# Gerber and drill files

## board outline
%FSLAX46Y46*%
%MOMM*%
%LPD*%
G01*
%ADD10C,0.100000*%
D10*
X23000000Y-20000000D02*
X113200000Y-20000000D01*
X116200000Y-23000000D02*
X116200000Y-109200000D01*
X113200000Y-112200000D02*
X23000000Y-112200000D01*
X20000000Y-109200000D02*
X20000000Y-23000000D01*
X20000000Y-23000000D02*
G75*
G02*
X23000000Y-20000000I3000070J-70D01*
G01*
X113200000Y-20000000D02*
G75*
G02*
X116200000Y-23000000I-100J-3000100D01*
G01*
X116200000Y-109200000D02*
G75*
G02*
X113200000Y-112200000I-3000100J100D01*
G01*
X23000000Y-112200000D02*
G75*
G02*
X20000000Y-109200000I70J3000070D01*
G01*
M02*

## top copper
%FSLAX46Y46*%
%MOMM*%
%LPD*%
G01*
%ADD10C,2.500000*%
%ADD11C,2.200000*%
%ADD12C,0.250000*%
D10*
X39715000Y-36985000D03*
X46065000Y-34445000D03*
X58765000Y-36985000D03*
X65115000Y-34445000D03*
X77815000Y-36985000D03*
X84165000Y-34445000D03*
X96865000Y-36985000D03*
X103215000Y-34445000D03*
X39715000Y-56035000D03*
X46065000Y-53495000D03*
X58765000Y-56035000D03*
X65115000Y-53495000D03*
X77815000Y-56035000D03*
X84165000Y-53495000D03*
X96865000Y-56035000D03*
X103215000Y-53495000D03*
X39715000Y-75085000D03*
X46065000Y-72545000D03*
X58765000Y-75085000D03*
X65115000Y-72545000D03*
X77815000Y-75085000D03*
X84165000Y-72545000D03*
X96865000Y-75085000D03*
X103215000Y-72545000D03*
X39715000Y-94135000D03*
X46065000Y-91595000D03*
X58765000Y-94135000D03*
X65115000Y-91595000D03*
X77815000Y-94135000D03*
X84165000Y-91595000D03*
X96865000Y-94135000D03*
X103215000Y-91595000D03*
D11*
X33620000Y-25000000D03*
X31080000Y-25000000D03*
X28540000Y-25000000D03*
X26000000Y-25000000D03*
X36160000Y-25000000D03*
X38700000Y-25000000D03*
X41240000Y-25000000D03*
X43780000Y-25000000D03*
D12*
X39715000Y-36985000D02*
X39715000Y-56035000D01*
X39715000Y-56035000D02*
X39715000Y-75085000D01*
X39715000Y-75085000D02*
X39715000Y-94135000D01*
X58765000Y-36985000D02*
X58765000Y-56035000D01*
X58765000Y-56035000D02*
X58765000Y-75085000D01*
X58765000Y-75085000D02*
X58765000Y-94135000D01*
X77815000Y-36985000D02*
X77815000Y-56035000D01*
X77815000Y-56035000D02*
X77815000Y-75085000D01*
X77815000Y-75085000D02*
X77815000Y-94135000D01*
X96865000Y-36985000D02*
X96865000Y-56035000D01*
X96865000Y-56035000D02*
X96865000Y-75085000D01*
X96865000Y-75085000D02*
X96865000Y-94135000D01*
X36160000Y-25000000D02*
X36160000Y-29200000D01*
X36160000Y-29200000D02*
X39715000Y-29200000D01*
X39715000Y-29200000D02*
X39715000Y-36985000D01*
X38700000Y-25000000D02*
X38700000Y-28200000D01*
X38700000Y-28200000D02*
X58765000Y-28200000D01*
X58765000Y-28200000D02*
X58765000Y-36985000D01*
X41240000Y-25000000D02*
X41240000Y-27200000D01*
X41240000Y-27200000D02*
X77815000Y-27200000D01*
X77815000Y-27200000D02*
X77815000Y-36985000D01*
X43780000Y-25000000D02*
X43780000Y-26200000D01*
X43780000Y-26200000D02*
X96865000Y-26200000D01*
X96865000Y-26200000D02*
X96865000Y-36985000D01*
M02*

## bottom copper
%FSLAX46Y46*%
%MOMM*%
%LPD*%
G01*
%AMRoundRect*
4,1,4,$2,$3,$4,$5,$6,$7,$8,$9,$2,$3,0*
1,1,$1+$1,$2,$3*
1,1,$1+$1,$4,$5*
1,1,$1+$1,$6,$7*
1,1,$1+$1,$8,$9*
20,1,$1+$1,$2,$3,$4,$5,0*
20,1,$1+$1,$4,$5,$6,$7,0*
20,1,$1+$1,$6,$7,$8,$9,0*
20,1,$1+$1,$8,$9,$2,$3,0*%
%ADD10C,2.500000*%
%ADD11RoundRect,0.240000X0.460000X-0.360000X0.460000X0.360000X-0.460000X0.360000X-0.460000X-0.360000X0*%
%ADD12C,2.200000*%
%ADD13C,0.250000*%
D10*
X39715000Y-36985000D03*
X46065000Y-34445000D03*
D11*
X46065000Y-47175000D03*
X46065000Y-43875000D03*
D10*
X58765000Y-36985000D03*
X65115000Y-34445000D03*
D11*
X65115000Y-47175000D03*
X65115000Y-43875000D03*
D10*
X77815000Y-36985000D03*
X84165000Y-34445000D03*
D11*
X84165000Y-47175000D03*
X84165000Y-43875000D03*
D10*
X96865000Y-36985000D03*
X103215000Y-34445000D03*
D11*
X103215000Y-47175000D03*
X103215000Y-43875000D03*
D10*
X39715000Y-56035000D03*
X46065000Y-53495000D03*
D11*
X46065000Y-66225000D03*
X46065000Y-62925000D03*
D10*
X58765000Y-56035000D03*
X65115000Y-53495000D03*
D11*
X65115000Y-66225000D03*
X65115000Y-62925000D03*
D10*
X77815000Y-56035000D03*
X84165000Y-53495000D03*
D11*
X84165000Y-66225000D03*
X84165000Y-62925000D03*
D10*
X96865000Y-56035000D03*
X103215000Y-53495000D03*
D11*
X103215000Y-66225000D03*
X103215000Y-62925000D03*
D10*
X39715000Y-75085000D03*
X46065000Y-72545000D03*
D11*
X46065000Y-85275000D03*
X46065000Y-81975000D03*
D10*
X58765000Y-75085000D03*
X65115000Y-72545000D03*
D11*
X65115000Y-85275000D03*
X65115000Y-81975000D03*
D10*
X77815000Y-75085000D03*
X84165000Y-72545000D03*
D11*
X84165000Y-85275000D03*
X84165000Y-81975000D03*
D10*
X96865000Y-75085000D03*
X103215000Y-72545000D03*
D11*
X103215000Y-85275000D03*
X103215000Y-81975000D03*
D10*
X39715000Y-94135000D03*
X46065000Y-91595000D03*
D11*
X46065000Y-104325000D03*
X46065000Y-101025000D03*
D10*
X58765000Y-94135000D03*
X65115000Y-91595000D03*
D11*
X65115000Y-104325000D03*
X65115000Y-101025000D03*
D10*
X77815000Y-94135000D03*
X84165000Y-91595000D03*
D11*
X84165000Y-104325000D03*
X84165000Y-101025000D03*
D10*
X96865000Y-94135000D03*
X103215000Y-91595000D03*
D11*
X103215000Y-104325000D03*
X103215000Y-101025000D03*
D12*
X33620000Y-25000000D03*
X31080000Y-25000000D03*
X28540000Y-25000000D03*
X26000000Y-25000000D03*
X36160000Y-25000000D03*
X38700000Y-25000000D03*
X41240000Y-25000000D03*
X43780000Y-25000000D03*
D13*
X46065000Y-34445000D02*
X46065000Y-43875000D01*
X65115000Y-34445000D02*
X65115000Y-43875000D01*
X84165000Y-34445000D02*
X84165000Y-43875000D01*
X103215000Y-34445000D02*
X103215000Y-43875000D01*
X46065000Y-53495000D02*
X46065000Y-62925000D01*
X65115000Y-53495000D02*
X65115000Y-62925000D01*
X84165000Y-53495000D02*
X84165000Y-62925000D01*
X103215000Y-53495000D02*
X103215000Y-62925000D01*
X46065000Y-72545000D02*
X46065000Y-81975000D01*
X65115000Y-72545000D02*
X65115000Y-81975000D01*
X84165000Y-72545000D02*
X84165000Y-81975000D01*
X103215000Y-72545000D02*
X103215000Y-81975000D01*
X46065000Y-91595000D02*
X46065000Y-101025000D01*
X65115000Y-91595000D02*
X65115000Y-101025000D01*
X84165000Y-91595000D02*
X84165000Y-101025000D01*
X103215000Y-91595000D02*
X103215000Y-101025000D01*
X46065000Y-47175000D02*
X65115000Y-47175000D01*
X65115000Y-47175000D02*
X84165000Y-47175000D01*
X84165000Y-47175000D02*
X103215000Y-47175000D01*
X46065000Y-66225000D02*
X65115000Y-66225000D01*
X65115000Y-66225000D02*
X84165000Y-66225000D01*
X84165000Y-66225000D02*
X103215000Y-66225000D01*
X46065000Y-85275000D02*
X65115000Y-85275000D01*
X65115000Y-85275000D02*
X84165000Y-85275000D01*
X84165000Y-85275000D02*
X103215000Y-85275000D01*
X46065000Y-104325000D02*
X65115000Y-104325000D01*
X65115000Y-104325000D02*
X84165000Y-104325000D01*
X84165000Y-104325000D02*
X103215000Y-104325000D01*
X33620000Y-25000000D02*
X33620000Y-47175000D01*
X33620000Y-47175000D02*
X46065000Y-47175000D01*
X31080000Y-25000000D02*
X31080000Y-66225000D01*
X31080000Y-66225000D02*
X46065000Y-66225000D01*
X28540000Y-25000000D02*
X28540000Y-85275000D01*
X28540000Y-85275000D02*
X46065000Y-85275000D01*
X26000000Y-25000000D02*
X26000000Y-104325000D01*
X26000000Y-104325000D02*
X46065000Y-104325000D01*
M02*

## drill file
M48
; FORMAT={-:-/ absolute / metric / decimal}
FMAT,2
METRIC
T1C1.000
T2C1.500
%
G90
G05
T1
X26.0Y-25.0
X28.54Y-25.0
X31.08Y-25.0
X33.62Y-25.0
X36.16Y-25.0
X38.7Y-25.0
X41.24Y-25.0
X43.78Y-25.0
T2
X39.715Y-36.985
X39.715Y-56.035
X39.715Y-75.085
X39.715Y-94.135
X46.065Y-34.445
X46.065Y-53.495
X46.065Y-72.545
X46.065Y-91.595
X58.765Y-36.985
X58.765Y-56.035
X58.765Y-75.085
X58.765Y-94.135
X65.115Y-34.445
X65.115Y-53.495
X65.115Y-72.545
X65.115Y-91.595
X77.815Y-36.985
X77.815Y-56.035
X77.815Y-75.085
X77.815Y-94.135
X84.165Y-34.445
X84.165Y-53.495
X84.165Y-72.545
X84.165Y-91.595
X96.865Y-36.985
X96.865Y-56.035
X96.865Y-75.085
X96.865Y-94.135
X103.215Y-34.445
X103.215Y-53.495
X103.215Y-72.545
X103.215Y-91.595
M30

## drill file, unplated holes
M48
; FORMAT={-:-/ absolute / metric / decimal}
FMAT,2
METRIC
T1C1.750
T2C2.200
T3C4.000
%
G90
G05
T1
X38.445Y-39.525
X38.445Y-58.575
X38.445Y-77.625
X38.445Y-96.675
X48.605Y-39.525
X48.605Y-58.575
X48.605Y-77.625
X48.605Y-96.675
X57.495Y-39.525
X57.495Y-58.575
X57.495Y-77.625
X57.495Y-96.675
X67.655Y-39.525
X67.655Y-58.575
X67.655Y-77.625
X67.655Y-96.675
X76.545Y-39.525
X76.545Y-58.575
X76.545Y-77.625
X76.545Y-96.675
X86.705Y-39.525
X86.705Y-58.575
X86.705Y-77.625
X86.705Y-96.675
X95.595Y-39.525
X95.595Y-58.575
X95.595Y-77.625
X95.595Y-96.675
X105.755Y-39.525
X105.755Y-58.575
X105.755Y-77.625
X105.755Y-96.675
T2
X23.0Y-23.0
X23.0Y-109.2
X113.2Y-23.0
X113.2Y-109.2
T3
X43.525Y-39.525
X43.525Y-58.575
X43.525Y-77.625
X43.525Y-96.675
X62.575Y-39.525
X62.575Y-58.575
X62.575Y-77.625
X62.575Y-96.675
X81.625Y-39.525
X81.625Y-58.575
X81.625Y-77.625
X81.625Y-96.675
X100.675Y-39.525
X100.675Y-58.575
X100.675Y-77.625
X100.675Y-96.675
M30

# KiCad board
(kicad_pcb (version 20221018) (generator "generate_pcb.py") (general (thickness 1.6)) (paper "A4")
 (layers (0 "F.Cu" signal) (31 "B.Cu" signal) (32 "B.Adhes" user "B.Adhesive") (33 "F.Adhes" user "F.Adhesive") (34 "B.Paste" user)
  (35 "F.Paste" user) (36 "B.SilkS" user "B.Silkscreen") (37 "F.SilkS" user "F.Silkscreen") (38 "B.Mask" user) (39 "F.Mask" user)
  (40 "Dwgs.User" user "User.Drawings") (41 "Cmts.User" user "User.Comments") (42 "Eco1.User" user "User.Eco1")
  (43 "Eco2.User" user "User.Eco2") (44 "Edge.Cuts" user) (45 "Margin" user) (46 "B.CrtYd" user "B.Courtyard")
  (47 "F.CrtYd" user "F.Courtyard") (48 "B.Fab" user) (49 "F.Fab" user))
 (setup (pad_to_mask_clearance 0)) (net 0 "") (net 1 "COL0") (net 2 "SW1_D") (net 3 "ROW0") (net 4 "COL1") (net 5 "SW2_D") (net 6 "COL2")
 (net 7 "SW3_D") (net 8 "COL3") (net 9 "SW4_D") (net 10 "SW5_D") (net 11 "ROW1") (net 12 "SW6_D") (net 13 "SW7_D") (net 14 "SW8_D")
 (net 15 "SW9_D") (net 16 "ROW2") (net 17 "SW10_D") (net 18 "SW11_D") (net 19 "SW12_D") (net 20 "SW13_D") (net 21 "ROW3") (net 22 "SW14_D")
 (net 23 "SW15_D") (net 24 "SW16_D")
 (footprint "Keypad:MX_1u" (layer "F.Cu") (at 43.5250 39.5250)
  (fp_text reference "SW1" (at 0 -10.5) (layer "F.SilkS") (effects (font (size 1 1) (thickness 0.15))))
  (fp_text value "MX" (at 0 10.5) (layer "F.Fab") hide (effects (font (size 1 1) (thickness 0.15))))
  (pad "1" thru_hole circle (at -3.81 -2.54) (size 2.5 2.5) (drill 1.5) (layers "*.Cu" "*.Mask") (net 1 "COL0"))
  (pad "2" thru_hole circle (at 2.54 -5.08) (size 2.5 2.5) (drill 1.5) (layers "*.Cu" "*.Mask") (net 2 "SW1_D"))
  (pad "" np_thru_hole circle (at 0 0) (size 4 4) (drill 4) (layers "*.Cu" "*.Mask"))
  (pad "" np_thru_hole circle (at -5.08 0) (size 1.75 1.75) (drill 1.75) (layers "*.Cu" "*.Mask"))
  (pad "" np_thru_hole circle (at 5.08 0) (size 1.75 1.75) (drill 1.75) (layers "*.Cu" "*.Mask")))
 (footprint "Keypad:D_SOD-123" (layer "B.Cu") (at 46.0650 45.5250 90)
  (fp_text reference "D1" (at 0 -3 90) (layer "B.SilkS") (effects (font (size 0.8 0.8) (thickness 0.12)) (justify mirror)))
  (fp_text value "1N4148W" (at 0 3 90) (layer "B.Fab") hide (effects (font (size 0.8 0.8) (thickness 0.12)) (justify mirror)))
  (pad "1" smd roundrect (at -1.65 0 90) (size 1.2 1.4) (layers "B.Cu" "B.Paste" "B.Mask") (roundrect_rratio 0.2) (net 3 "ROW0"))
  (pad "2" smd roundrect (at 1.65 0 90) (size 1.2 1.4) (layers "B.Cu" "B.Paste" "B.Mask") (roundrect_rratio 0.2) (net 2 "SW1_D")))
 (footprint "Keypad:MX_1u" (layer "F.Cu") (at 62.5750 39.5250)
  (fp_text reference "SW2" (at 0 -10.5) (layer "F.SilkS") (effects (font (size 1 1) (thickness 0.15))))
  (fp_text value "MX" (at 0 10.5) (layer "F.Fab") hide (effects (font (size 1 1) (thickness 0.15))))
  (pad "1" thru_hole circle (at -3.81 -2.54) (size 2.5 2.5) (drill 1.5) (layers "*.Cu" "*.Mask") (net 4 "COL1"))
  (pad "2" thru_hole circle (at 2.54 -5.08) (size 2.5 2.5) (drill 1.5) (layers "*.Cu" "*.Mask") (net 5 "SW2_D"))
  (pad "" np_thru_hole circle (at 0 0) (size 4 4) (drill 4) (layers "*.Cu" "*.Mask"))
  (pad "" np_thru_hole circle (at -5.08 0) (size 1.75 1.75) (drill 1.75) (layers "*.Cu" "*.Mask"))
  (pad "" np_thru_hole circle (at 5.08 0) (size 1.75 1.75) (drill 1.75) (layers "*.Cu" "*.Mask")))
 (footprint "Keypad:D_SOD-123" (layer "B.Cu") (at 65.1150 45.5250 90)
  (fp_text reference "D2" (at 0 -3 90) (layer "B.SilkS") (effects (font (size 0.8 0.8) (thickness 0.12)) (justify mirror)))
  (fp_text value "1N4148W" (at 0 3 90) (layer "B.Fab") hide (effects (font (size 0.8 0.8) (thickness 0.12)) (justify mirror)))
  (pad "1" smd roundrect (at -1.65 0 90) (size 1.2 1.4) (layers "B.Cu" "B.Paste" "B.Mask") (roundrect_rratio 0.2) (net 3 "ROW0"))
  (pad "2" smd roundrect (at 1.65 0 90) (size 1.2 1.4) (layers "B.Cu" "B.Paste" "B.Mask") (roundrect_rratio 0.2) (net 5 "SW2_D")))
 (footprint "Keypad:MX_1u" (layer "F.Cu") (at 81.6250 39.5250)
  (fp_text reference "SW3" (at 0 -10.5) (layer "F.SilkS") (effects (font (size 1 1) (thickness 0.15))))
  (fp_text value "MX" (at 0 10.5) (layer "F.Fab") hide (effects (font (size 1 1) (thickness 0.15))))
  (pad "1" thru_hole circle (at -3.81 -2.54) (size 2.5 2.5) (drill 1.5) (layers "*.Cu" "*.Mask") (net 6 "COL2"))
  (pad "2" thru_hole circle (at 2.54 -5.08) (size 2.5 2.5) (drill 1.5) (layers "*.Cu" "*.Mask") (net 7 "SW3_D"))
  (pad "" np_thru_hole circle (at 0 0) (size 4 4) (drill 4) (layers "*.Cu" "*.Mask"))
  (pad "" np_thru_hole circle (at -5.08 0) (size 1.75 1.75) (drill 1.75) (layers "*.Cu" "*.Mask"))
  (pad "" np_thru_hole circle (at 5.08 0) (size 1.75 1.75) (drill 1.75) (layers "*.Cu" "*.Mask")))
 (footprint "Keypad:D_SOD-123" (layer "B.Cu") (at 84.1650 45.5250 90)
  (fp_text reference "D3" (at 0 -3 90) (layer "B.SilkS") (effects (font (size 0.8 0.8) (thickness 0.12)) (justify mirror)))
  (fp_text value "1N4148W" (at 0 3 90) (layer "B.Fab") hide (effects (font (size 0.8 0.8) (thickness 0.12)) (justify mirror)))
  (pad "1" smd roundrect (at -1.65 0 90) (size 1.2 1.4) (layers "B.Cu" "B.Paste" "B.Mask") (roundrect_rratio 0.2) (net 3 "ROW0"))
  (pad "2" smd roundrect (at 1.65 0 90) (size 1.2 1.4) (layers "B.Cu" "B.Paste" "B.Mask") (roundrect_rratio 0.2) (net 7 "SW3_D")))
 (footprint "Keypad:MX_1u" (layer "F.Cu") (at 100.6750 39.5250)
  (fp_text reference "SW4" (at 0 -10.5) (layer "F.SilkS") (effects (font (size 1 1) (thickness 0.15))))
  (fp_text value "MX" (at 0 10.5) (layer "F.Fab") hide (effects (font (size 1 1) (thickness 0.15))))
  (pad "1" thru_hole circle (at -3.81 -2.54) (size 2.5 2.5) (drill 1.5) (layers "*.Cu" "*.Mask") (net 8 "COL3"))
  (pad "2" thru_hole circle (at 2.54 -5.08) (size 2.5 2.5) (drill 1.5) (layers "*.Cu" "*.Mask") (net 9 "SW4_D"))
  (pad "" np_thru_hole circle (at 0 0) (size 4 4) (drill 4) (layers "*.Cu" "*.Mask"))
  (pad "" np_thru_hole circle (at -5.08 0) (size 1.75 1.75) (drill 1.75) (layers "*.Cu" "*.Mask"))
  (pad "" np_thru_hole circle (at 5.08 0) (size 1.75 1.75) (drill 1.75) (layers "*.Cu" "*.Mask")))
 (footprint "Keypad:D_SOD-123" (layer "B.Cu") (at 103.2150 45.5250 90)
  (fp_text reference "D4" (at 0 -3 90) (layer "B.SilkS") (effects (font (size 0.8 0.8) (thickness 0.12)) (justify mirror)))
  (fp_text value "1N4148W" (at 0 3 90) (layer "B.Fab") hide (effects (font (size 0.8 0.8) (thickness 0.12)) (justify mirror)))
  (pad "1" smd roundrect (at -1.65 0 90) (size 1.2 1.4) (layers "B.Cu" "B.Paste" "B.Mask") (roundrect_rratio 0.2) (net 3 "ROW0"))
  (pad "2" smd roundrect (at 1.65 0 90) (size 1.2 1.4) (layers "B.Cu" "B.Paste" "B.Mask") (roundrect_rratio 0.2) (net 9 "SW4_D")))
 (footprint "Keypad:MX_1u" (layer "F.Cu") (at 43.5250 58.5750)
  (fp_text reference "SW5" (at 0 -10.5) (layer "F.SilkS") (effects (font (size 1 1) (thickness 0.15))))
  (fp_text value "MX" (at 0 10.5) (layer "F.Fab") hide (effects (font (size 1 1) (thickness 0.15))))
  (pad "1" thru_hole circle (at -3.81 -2.54) (size 2.5 2.5) (drill 1.5) (layers "*.Cu" "*.Mask") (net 1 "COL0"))
  (pad "2" thru_hole circle (at 2.54 -5.08) (size 2.5 2.5) (drill 1.5) (layers "*.Cu" "*.Mask") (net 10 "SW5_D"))
  (pad "" np_thru_hole circle (at 0 0) (size 4 4) (drill 4) (layers "*.Cu" "*.Mask"))
  (pad "" np_thru_hole circle (at -5.08 0) (size 1.75 1.75) (drill 1.75) (layers "*.Cu" "*.Mask"))
  (pad "" np_thru_hole circle (at 5.08 0) (size 1.75 1.75) (drill 1.75) (layers "*.Cu" "*.Mask")))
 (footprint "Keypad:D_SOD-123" (layer "B.Cu") (at 46.0650 64.5750 90)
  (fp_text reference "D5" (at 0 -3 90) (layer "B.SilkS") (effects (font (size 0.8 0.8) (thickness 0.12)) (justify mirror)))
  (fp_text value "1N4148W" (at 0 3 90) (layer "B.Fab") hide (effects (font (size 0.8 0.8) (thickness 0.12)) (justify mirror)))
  (pad "1" smd roundrect (at -1.65 0 90) (size 1.2 1.4) (layers "B.Cu" "B.Paste" "B.Mask") (roundrect_rratio 0.2) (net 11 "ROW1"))
  (pad "2" smd roundrect (at 1.65 0 90) (size 1.2 1.4) (layers "B.Cu" "B.Paste" "B.Mask") (roundrect_rratio 0.2) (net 10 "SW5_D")))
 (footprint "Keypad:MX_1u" (layer "F.Cu") (at 62.5750 58.5750)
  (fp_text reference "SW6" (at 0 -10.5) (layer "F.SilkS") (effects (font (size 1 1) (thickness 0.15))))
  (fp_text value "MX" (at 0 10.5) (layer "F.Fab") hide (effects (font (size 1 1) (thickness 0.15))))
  (pad "1" thru_hole circle (at -3.81 -2.54) (size 2.5 2.5) (drill 1.5) (layers "*.Cu" "*.Mask") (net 4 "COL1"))
  (pad "2" thru_hole circle (at 2.54 -5.08) (size 2.5 2.5) (drill 1.5) (layers "*.Cu" "*.Mask") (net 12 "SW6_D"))
  (pad "" np_thru_hole circle (at 0 0) (size 4 4) (drill 4) (layers "*.Cu" "*.Mask"))
  (pad "" np_thru_hole circle (at -5.08 0) (size 1.75 1.75) (drill 1.75) (layers "*.Cu" "*.Mask"))
  (pad "" np_thru_hole circle (at 5.08 0) (size 1.75 1.75) (drill 1.75) (layers "*.Cu" "*.Mask")))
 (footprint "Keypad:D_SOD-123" (layer "B.Cu") (at 65.1150 64.5750 90)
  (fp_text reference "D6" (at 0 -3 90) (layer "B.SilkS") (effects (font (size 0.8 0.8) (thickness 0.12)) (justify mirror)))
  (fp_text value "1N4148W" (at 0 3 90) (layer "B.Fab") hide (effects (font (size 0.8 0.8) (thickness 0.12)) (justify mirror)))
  (pad "1" smd roundrect (at -1.65 0 90) (size 1.2 1.4) (layers "B.Cu" "B.Paste" "B.Mask") (roundrect_rratio 0.2) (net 11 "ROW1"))
  (pad "2" smd roundrect (at 1.65 0 90) (size 1.2 1.4) (layers "B.Cu" "B.Paste" "B.Mask") (roundrect_rratio 0.2) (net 12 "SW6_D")))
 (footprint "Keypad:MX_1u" (layer "F.Cu") (at 81.6250 58.5750)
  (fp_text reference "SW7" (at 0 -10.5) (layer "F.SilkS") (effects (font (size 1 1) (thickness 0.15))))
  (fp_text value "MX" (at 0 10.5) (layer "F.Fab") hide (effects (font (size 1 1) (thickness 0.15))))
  (pad "1" thru_hole circle (at -3.81 -2.54) (size 2.5 2.5) (drill 1.5) (layers "*.Cu" "*.Mask") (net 6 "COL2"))
  (pad "2" thru_hole circle (at 2.54 -5.08) (size 2.5 2.5) (drill 1.5) (layers "*.Cu" "*.Mask") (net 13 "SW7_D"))
  (pad "" np_thru_hole circle (at 0 0) (size 4 4) (drill 4) (layers "*.Cu" "*.Mask"))
  (pad "" np_thru_hole circle (at -5.08 0) (size 1.75 1.75) (drill 1.75) (layers "*.Cu" "*.Mask"))
  (pad "" np_thru_hole circle (at 5.08 0) (size 1.75 1.75) (drill 1.75) (layers "*.Cu" "*.Mask")))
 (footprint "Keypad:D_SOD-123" (layer "B.Cu") (at 84.1650 64.5750 90)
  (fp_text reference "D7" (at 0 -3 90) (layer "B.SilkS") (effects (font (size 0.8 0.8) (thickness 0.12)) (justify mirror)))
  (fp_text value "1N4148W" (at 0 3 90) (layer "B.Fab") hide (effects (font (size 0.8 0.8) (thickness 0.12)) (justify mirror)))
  (pad "1" smd roundrect (at -1.65 0 90) (size 1.2 1.4) (layers "B.Cu" "B.Paste" "B.Mask") (roundrect_rratio 0.2) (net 11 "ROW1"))
  (pad "2" smd roundrect (at 1.65 0 90) (size 1.2 1.4) (layers "B.Cu" "B.Paste" "B.Mask") (roundrect_rratio 0.2) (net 13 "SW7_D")))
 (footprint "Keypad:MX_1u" (layer "F.Cu") (at 100.6750 58.5750)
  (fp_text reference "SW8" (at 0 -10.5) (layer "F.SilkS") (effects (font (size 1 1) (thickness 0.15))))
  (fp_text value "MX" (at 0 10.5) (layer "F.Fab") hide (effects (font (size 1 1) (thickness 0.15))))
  (pad "1" thru_hole circle (at -3.81 -2.54) (size 2.5 2.5) (drill 1.5) (layers "*.Cu" "*.Mask") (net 8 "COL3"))
  (pad "2" thru_hole circle (at 2.54 -5.08) (size 2.5 2.5) (drill 1.5) (layers "*.Cu" "*.Mask") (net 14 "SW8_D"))
  (pad "" np_thru_hole circle (at 0 0) (size 4 4) (drill 4) (layers "*.Cu" "*.Mask"))
  (pad "" np_thru_hole circle (at -5.08 0) (size 1.75 1.75) (drill 1.75) (layers "*.Cu" "*.Mask"))
  (pad "" np_thru_hole circle (at 5.08 0) (size 1.75 1.75) (drill 1.75) (layers "*.Cu" "*.Mask")))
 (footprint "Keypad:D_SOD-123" (layer "B.Cu") (at 103.2150 64.5750 90)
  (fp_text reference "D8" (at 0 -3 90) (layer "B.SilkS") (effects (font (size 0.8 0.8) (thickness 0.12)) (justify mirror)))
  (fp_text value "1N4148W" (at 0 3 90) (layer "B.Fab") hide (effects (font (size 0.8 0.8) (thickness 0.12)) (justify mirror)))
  (pad "1" smd roundrect (at -1.65 0 90) (size 1.2 1.4) (layers "B.Cu" "B.Paste" "B.Mask") (roundrect_rratio 0.2) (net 11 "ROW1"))
  (pad "2" smd roundrect (at 1.65 0 90) (size 1.2 1.4) (layers "B.Cu" "B.Paste" "B.Mask") (roundrect_rratio 0.2) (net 14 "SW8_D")))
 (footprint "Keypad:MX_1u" (layer "F.Cu") (at 43.5250 77.6250)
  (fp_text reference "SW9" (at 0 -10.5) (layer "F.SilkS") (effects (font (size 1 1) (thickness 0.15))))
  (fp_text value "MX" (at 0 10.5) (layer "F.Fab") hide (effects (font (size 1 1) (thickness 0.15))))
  (pad "1" thru_hole circle (at -3.81 -2.54) (size 2.5 2.5) (drill 1.5) (layers "*.Cu" "*.Mask") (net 1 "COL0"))
  (pad "2" thru_hole circle (at 2.54 -5.08) (size 2.5 2.5) (drill 1.5) (layers "*.Cu" "*.Mask") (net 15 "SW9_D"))
  (pad "" np_thru_hole circle (at 0 0) (size 4 4) (drill 4) (layers "*.Cu" "*.Mask"))
  (pad "" np_thru_hole circle (at -5.08 0) (size 1.75 1.75) (drill 1.75) (layers "*.Cu" "*.Mask"))
  (pad "" np_thru_hole circle (at 5.08 0) (size 1.75 1.75) (drill 1.75) (layers "*.Cu" "*.Mask")))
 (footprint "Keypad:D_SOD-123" (layer "B.Cu") (at 46.0650 83.6250 90)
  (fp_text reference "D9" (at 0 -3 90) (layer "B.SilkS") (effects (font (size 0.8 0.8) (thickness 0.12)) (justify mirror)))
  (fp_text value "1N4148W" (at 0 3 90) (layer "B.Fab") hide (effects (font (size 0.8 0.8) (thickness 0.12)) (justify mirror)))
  (pad "1" smd roundrect (at -1.65 0 90) (size 1.2 1.4) (layers "B.Cu" "B.Paste" "B.Mask") (roundrect_rratio 0.2) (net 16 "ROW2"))
  (pad "2" smd roundrect (at 1.65 0 90) (size 1.2 1.4) (layers "B.Cu" "B.Paste" "B.Mask") (roundrect_rratio 0.2) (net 15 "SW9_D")))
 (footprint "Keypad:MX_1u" (layer "F.Cu") (at 62.5750 77.6250)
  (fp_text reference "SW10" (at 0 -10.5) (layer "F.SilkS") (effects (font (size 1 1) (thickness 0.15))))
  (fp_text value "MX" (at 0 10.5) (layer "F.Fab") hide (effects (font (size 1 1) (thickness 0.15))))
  (pad "1" thru_hole circle (at -3.81 -2.54) (size 2.5 2.5) (drill 1.5) (layers "*.Cu" "*.Mask") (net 4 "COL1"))
  (pad "2" thru_hole circle (at 2.54 -5.08) (size 2.5 2.5) (drill 1.5) (layers "*.Cu" "*.Mask") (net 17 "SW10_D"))
  (pad "" np_thru_hole circle (at 0 0) (size 4 4) (drill 4) (layers "*.Cu" "*.Mask"))
  (pad "" np_thru_hole circle (at -5.08 0) (size 1.75 1.75) (drill 1.75) (layers "*.Cu" "*.Mask"))
  (pad "" np_thru_hole circle (at 5.08 0) (size 1.75 1.75) (drill 1.75) (layers "*.Cu" "*.Mask")))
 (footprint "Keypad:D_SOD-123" (layer "B.Cu") (at 65.1150 83.6250 90)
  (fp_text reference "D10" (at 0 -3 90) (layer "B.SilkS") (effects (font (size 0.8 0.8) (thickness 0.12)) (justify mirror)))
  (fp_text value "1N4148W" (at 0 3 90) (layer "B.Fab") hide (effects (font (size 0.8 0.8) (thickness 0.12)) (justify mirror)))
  (pad "1" smd roundrect (at -1.65 0 90) (size 1.2 1.4) (layers "B.Cu" "B.Paste" "B.Mask") (roundrect_rratio 0.2) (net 16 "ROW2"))
  (pad "2" smd roundrect (at 1.65 0 90) (size 1.2 1.4) (layers "B.Cu" "B.Paste" "B.Mask") (roundrect_rratio 0.2) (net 17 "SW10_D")))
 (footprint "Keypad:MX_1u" (layer "F.Cu") (at 81.6250 77.6250)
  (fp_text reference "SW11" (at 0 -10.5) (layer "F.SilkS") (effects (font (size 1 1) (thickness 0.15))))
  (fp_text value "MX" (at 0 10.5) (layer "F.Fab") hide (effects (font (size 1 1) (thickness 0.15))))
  (pad "1" thru_hole circle (at -3.81 -2.54) (size 2.5 2.5) (drill 1.5) (layers "*.Cu" "*.Mask") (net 6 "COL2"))
  (pad "2" thru_hole circle (at 2.54 -5.08) (size 2.5 2.5) (drill 1.5) (layers "*.Cu" "*.Mask") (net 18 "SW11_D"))
  (pad "" np_thru_hole circle (at 0 0) (size 4 4) (drill 4) (layers "*.Cu" "*.Mask"))
  (pad "" np_thru_hole circle (at -5.08 0) (size 1.75 1.75) (drill 1.75) (layers "*.Cu" "*.Mask"))
  (pad "" np_thru_hole circle (at 5.08 0) (size 1.75 1.75) (drill 1.75) (layers "*.Cu" "*.Mask")))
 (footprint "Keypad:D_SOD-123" (layer "B.Cu") (at 84.1650 83.6250 90)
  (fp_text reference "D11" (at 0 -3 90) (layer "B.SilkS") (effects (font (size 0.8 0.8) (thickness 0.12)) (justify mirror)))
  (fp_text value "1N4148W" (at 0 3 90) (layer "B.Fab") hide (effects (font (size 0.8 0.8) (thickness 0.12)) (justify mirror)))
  (pad "1" smd roundrect (at -1.65 0 90) (size 1.2 1.4) (layers "B.Cu" "B.Paste" "B.Mask") (roundrect_rratio 0.2) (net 16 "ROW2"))
  (pad "2" smd roundrect (at 1.65 0 90) (size 1.2 1.4) (layers "B.Cu" "B.Paste" "B.Mask") (roundrect_rratio 0.2) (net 18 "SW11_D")))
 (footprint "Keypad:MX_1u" (layer "F.Cu") (at 100.6750 77.6250)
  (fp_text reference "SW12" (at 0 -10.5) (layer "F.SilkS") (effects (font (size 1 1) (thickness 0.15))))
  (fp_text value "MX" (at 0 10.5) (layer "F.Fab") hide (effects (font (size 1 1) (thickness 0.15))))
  (pad "1" thru_hole circle (at -3.81 -2.54) (size 2.5 2.5) (drill 1.5) (layers "*.Cu" "*.Mask") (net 8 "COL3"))
  (pad "2" thru_hole circle (at 2.54 -5.08) (size 2.5 2.5) (drill 1.5) (layers "*.Cu" "*.Mask") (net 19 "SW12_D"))
  (pad "" np_thru_hole circle (at 0 0) (size 4 4) (drill 4) (layers "*.Cu" "*.Mask"))
  (pad "" np_thru_hole circle (at -5.08 0) (size 1.75 1.75) (drill 1.75) (layers "*.Cu" "*.Mask"))
  (pad "" np_thru_hole circle (at 5.08 0) (size 1.75 1.75) (drill 1.75) (layers "*.Cu" "*.Mask")))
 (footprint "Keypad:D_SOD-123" (layer "B.Cu") (at 103.2150 83.6250 90)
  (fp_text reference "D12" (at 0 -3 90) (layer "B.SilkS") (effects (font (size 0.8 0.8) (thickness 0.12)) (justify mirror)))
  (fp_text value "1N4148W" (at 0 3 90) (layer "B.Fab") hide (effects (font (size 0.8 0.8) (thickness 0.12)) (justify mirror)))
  (pad "1" smd roundrect (at -1.65 0 90) (size 1.2 1.4) (layers "B.Cu" "B.Paste" "B.Mask") (roundrect_rratio 0.2) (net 16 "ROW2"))
  (pad "2" smd roundrect (at 1.65 0 90) (size 1.2 1.4) (layers "B.Cu" "B.Paste" "B.Mask") (roundrect_rratio 0.2) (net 19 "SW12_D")))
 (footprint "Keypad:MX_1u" (layer "F.Cu") (at 43.5250 96.6750)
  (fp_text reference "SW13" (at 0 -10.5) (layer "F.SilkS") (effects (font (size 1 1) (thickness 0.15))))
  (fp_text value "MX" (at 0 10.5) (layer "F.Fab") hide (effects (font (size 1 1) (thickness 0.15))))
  (pad "1" thru_hole circle (at -3.81 -2.54) (size 2.5 2.5) (drill 1.5) (layers "*.Cu" "*.Mask") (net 1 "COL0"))
  (pad "2" thru_hole circle (at 2.54 -5.08) (size 2.5 2.5) (drill 1.5) (layers "*.Cu" "*.Mask") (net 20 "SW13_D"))
  (pad "" np_thru_hole circle (at 0 0) (size 4 4) (drill 4) (layers "*.Cu" "*.Mask"))
  (pad "" np_thru_hole circle (at -5.08 0) (size 1.75 1.75) (drill 1.75) (layers "*.Cu" "*.Mask"))
  (pad "" np_thru_hole circle (at 5.08 0) (size 1.75 1.75) (drill 1.75) (layers "*.Cu" "*.Mask")))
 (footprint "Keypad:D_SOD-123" (layer "B.Cu") (at 46.0650 102.6750 90)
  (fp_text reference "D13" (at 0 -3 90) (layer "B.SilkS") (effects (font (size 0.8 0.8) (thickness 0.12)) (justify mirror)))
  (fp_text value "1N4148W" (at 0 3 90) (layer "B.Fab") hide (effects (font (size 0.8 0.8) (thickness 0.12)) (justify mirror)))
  (pad "1" smd roundrect (at -1.65 0 90) (size 1.2 1.4) (layers "B.Cu" "B.Paste" "B.Mask") (roundrect_rratio 0.2) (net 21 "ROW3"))
  (pad "2" smd roundrect (at 1.65 0 90) (size 1.2 1.4) (layers "B.Cu" "B.Paste" "B.Mask") (roundrect_rratio 0.2) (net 20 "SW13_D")))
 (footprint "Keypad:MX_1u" (layer "F.Cu") (at 62.5750 96.6750)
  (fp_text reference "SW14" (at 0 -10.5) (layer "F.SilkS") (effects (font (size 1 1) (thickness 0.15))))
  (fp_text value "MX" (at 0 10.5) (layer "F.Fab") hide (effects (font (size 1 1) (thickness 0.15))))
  (pad "1" thru_hole circle (at -3.81 -2.54) (size 2.5 2.5) (drill 1.5) (layers "*.Cu" "*.Mask") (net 4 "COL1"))
  (pad "2" thru_hole circle (at 2.54 -5.08) (size 2.5 2.5) (drill 1.5) (layers "*.Cu" "*.Mask") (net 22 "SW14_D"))
  (pad "" np_thru_hole circle (at 0 0) (size 4 4) (drill 4) (layers "*.Cu" "*.Mask"))
  (pad "" np_thru_hole circle (at -5.08 0) (size 1.75 1.75) (drill 1.75) (layers "*.Cu" "*.Mask"))
  (pad "" np_thru_hole circle (at 5.08 0) (size 1.75 1.75) (drill 1.75) (layers "*.Cu" "*.Mask")))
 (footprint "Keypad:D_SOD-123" (layer "B.Cu") (at 65.1150 102.6750 90)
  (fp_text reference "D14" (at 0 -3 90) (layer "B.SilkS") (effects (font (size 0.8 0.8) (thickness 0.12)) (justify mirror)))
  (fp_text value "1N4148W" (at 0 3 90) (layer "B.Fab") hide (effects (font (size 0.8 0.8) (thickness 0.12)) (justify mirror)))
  (pad "1" smd roundrect (at -1.65 0 90) (size 1.2 1.4) (layers "B.Cu" "B.Paste" "B.Mask") (roundrect_rratio 0.2) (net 21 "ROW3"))
  (pad "2" smd roundrect (at 1.65 0 90) (size 1.2 1.4) (layers "B.Cu" "B.Paste" "B.Mask") (roundrect_rratio 0.2) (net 22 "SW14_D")))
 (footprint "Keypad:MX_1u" (layer "F.Cu") (at 81.6250 96.6750)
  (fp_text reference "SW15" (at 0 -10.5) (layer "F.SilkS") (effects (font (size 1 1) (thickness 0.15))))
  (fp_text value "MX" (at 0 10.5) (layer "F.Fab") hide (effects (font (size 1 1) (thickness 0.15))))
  (pad "1" thru_hole circle (at -3.81 -2.54) (size 2.5 2.5) (drill 1.5) (layers "*.Cu" "*.Mask") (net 6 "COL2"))
  (pad "2" thru_hole circle (at 2.54 -5.08) (size 2.5 2.5) (drill 1.5) (layers "*.Cu" "*.Mask") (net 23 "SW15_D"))
  (pad "" np_thru_hole circle (at 0 0) (size 4 4) (drill 4) (layers "*.Cu" "*.Mask"))
  (pad "" np_thru_hole circle (at -5.08 0) (size 1.75 1.75) (drill 1.75) (layers "*.Cu" "*.Mask"))
  (pad "" np_thru_hole circle (at 5.08 0) (size 1.75 1.75) (drill 1.75) (layers "*.Cu" "*.Mask")))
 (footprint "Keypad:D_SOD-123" (layer "B.Cu") (at 84.1650 102.6750 90)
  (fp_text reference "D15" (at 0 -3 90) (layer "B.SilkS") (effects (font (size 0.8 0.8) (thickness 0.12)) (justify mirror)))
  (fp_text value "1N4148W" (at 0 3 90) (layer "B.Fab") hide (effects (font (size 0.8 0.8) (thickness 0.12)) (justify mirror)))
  (pad "1" smd roundrect (at -1.65 0 90) (size 1.2 1.4) (layers "B.Cu" "B.Paste" "B.Mask") (roundrect_rratio 0.2) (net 21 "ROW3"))
  (pad "2" smd roundrect (at 1.65 0 90) (size 1.2 1.4) (layers "B.Cu" "B.Paste" "B.Mask") (roundrect_rratio 0.2) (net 23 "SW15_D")))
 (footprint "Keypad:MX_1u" (layer "F.Cu") (at 100.6750 96.6750)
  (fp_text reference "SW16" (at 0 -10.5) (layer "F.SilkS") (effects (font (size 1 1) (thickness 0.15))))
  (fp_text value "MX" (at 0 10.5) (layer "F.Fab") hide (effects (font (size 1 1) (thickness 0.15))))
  (pad "1" thru_hole circle (at -3.81 -2.54) (size 2.5 2.5) (drill 1.5) (layers "*.Cu" "*.Mask") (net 8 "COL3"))
  (pad "2" thru_hole circle (at 2.54 -5.08) (size 2.5 2.5) (drill 1.5) (layers "*.Cu" "*.Mask") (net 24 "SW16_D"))
  (pad "" np_thru_hole circle (at 0 0) (size 4 4) (drill 4) (layers "*.Cu" "*.Mask"))
  (pad "" np_thru_hole circle (at -5.08 0) (size 1.75 1.75) (drill 1.75) (layers "*.Cu" "*.Mask"))
  (pad "" np_thru_hole circle (at 5.08 0) (size 1.75 1.75) (drill 1.75) (layers "*.Cu" "*.Mask")))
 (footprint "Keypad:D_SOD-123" (layer "B.Cu") (at 103.2150 102.6750 90)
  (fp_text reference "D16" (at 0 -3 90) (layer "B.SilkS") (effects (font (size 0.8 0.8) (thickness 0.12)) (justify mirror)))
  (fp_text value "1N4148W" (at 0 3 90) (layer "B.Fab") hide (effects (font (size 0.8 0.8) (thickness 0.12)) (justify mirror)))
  (pad "1" smd roundrect (at -1.65 0 90) (size 1.2 1.4) (layers "B.Cu" "B.Paste" "B.Mask") (roundrect_rratio 0.2) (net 21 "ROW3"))
  (pad "2" smd roundrect (at 1.65 0 90) (size 1.2 1.4) (layers "B.Cu" "B.Paste" "B.Mask") (roundrect_rratio 0.2) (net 24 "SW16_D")))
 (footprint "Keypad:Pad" (layer "F.Cu") (at 33.6200 25.0000)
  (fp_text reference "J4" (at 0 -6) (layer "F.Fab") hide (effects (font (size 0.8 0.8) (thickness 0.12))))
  (pad "1" thru_hole circle (at 0 0) (size 2.2 2.2) (drill 1.0) (layers "*.Cu" "*.Mask") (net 3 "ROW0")))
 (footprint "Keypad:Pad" (layer "F.Cu") (at 31.0800 25.0000)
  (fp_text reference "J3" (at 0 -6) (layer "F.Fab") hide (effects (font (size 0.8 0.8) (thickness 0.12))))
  (pad "1" thru_hole circle (at 0 0) (size 2.2 2.2) (drill 1.0) (layers "*.Cu" "*.Mask") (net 11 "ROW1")))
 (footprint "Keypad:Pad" (layer "F.Cu") (at 28.5400 25.0000)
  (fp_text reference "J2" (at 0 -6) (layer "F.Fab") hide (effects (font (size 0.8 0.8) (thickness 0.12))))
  (pad "1" thru_hole circle (at 0 0) (size 2.2 2.2) (drill 1.0) (layers "*.Cu" "*.Mask") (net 16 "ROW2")))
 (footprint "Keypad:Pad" (layer "F.Cu") (at 26.0000 25.0000)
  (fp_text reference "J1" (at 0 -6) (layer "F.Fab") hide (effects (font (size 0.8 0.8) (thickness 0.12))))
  (pad "1" thru_hole circle (at 0 0) (size 2.2 2.2) (drill 1.0) (layers "*.Cu" "*.Mask") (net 21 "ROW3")))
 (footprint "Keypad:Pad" (layer "F.Cu") (at 36.1600 25.0000)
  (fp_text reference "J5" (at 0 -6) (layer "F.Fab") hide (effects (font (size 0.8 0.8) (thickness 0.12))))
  (pad "1" thru_hole circle (at 0 0) (size 2.2 2.2) (drill 1.0) (layers "*.Cu" "*.Mask") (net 1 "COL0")))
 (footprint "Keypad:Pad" (layer "F.Cu") (at 38.7000 25.0000)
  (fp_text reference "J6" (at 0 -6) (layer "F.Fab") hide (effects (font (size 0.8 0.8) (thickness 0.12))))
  (pad "1" thru_hole circle (at 0 0) (size 2.2 2.2) (drill 1.0) (layers "*.Cu" "*.Mask") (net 4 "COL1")))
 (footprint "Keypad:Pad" (layer "F.Cu") (at 41.2400 25.0000)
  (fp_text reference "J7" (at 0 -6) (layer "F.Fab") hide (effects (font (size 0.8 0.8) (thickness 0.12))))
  (pad "1" thru_hole circle (at 0 0) (size 2.2 2.2) (drill 1.0) (layers "*.Cu" "*.Mask") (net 6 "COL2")))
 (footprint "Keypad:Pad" (layer "F.Cu") (at 43.7800 25.0000)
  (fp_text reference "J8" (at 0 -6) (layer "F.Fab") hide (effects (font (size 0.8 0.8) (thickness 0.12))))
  (pad "1" thru_hole circle (at 0 0) (size 2.2 2.2) (drill 1.0) (layers "*.Cu" "*.Mask") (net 8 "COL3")))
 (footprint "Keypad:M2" (layer "F.Cu") (at 23.0000 23.0000)
  (pad "" np_thru_hole circle (at 0 0) (size 2.2 2.2) (drill 2.2) (layers "*.Cu" "*.Mask")))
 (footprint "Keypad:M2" (layer "F.Cu") (at 113.2000 23.0000)
  (pad "" np_thru_hole circle (at 0 0) (size 2.2 2.2) (drill 2.2) (layers "*.Cu" "*.Mask")))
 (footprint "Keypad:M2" (layer "F.Cu") (at 23.0000 109.2000)
  (pad "" np_thru_hole circle (at 0 0) (size 2.2 2.2) (drill 2.2) (layers "*.Cu" "*.Mask")))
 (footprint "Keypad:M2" (layer "F.Cu") (at 113.2000 109.2000)
  (pad "" np_thru_hole circle (at 0 0) (size 2.2 2.2) (drill 2.2) (layers "*.Cu" "*.Mask")))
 (segment (start 39.7150 36.9850) (end 39.7150 56.0350) (width 0.25) (layer "F.Cu") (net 1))
 (segment (start 39.7150 56.0350) (end 39.7150 75.0850) (width 0.25) (layer "F.Cu") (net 1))
 (segment (start 39.7150 75.0850) (end 39.7150 94.1350) (width 0.25) (layer "F.Cu") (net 1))
 (segment (start 58.7650 36.9850) (end 58.7650 56.0350) (width 0.25) (layer "F.Cu") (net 4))
 (segment (start 58.7650 56.0350) (end 58.7650 75.0850) (width 0.25) (layer "F.Cu") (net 4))
 (segment (start 58.7650 75.0850) (end 58.7650 94.1350) (width 0.25) (layer "F.Cu") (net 4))
 (segment (start 77.8150 36.9850) (end 77.8150 56.0350) (width 0.25) (layer "F.Cu") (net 6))
 (segment (start 77.8150 56.0350) (end 77.8150 75.0850) (width 0.25) (layer "F.Cu") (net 6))
 (segment (start 77.8150 75.0850) (end 77.8150 94.1350) (width 0.25) (layer "F.Cu") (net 6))
 (segment (start 96.8650 36.9850) (end 96.8650 56.0350) (width 0.25) (layer "F.Cu") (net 8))
 (segment (start 96.8650 56.0350) (end 96.8650 75.0850) (width 0.25) (layer "F.Cu") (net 8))
 (segment (start 96.8650 75.0850) (end 96.8650 94.1350) (width 0.25) (layer "F.Cu") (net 8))
 (segment (start 46.0650 34.4450) (end 46.0650 43.8750) (width 0.25) (layer "B.Cu") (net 2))
 (segment (start 65.1150 34.4450) (end 65.1150 43.8750) (width 0.25) (layer "B.Cu") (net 5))
 (segment (start 84.1650 34.4450) (end 84.1650 43.8750) (width 0.25) (layer "B.Cu") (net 7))
 (segment (start 103.2150 34.4450) (end 103.2150 43.8750) (width 0.25) (layer "B.Cu") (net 9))
 (segment (start 46.0650 53.4950) (end 46.0650 62.9250) (width 0.25) (layer "B.Cu") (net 10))
 (segment (start 65.1150 53.4950) (end 65.1150 62.9250) (width 0.25) (layer "B.Cu") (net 12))
 (segment (start 84.1650 53.4950) (end 84.1650 62.9250) (width 0.25) (layer "B.Cu") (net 13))
 (segment (start 103.2150 53.4950) (end 103.2150 62.9250) (width 0.25) (layer "B.Cu") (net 14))
 (segment (start 46.0650 72.5450) (end 46.0650 81.9750) (width 0.25) (layer "B.Cu") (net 15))
 (segment (start 65.1150 72.5450) (end 65.1150 81.9750) (width 0.25) (layer "B.Cu") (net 17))
 (segment (start 84.1650 72.5450) (end 84.1650 81.9750) (width 0.25) (layer "B.Cu") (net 18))
 (segment (start 103.2150 72.5450) (end 103.2150 81.9750) (width 0.25) (layer "B.Cu") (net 19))
 (segment (start 46.0650 91.5950) (end 46.0650 101.0250) (width 0.25) (layer "B.Cu") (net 20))
 (segment (start 65.1150 91.5950) (end 65.1150 101.0250) (width 0.25) (layer "B.Cu") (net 22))
 (segment (start 84.1650 91.5950) (end 84.1650 101.0250) (width 0.25) (layer "B.Cu") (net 23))
 (segment (start 103.2150 91.5950) (end 103.2150 101.0250) (width 0.25) (layer "B.Cu") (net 24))
 (segment (start 46.0650 47.1750) (end 65.1150 47.1750) (width 0.25) (layer "B.Cu") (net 3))
 (segment (start 65.1150 47.1750) (end 84.1650 47.1750) (width 0.25) (layer "B.Cu") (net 3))
 (segment (start 84.1650 47.1750) (end 103.2150 47.1750) (width 0.25) (layer "B.Cu") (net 3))
 (segment (start 46.0650 66.2250) (end 65.1150 66.2250) (width 0.25) (layer "B.Cu") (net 11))
 (segment (start 65.1150 66.2250) (end 84.1650 66.2250) (width 0.25) (layer "B.Cu") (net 11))
 (segment (start 84.1650 66.2250) (end 103.2150 66.2250) (width 0.25) (layer "B.Cu") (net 11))
 (segment (start 46.0650 85.2750) (end 65.1150 85.2750) (width 0.25) (layer "B.Cu") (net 16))
 (segment (start 65.1150 85.2750) (end 84.1650 85.2750) (width 0.25) (layer "B.Cu") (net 16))
 (segment (start 84.1650 85.2750) (end 103.2150 85.2750) (width 0.25) (layer "B.Cu") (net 16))
 (segment (start 46.0650 104.3250) (end 65.1150 104.3250) (width 0.25) (layer "B.Cu") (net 21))
 (segment (start 65.1150 104.3250) (end 84.1650 104.3250) (width 0.25) (layer "B.Cu") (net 21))
 (segment (start 84.1650 104.3250) (end 103.2150 104.3250) (width 0.25) (layer "B.Cu") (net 21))
 (segment (start 33.6200 25.0000) (end 33.6200 47.1750) (width 0.25) (layer "B.Cu") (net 3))
 (segment (start 33.6200 47.1750) (end 46.0650 47.1750) (width 0.25) (layer "B.Cu") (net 3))
 (segment (start 31.0800 25.0000) (end 31.0800 66.2250) (width 0.25) (layer "B.Cu") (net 11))
 (segment (start 31.0800 66.2250) (end 46.0650 66.2250) (width 0.25) (layer "B.Cu") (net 11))
 (segment (start 28.5400 25.0000) (end 28.5400 85.2750) (width 0.25) (layer "B.Cu") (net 16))
 (segment (start 28.5400 85.2750) (end 46.0650 85.2750) (width 0.25) (layer "B.Cu") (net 16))
 (segment (start 26.0000 25.0000) (end 26.0000 104.3250) (width 0.25) (layer "B.Cu") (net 21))
 (segment (start 26.0000 104.3250) (end 46.0650 104.3250) (width 0.25) (layer "B.Cu") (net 21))
 (segment (start 36.1600 25.0000) (end 36.1600 29.2000) (width 0.25) (layer "F.Cu") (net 1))
 (segment (start 36.1600 29.2000) (end 39.7150 29.2000) (width 0.25) (layer "F.Cu") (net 1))
 (segment (start 39.7150 29.2000) (end 39.7150 36.9850) (width 0.25) (layer "F.Cu") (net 1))
 (segment (start 38.7000 25.0000) (end 38.7000 28.2000) (width 0.25) (layer "F.Cu") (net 4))
 (segment (start 38.7000 28.2000) (end 58.7650 28.2000) (width 0.25) (layer "F.Cu") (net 4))
 (segment (start 58.7650 28.2000) (end 58.7650 36.9850) (width 0.25) (layer "F.Cu") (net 4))
 (segment (start 41.2400 25.0000) (end 41.2400 27.2000) (width 0.25) (layer "F.Cu") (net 6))
 (segment (start 41.2400 27.2000) (end 77.8150 27.2000) (width 0.25) (layer "F.Cu") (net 6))
 (segment (start 77.8150 27.2000) (end 77.8150 36.9850) (width 0.25) (layer "F.Cu") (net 6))
 (segment (start 43.7800 25.0000) (end 43.7800 26.2000) (width 0.25) (layer "F.Cu") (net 8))
 (segment (start 43.7800 26.2000) (end 96.8650 26.2000) (width 0.25) (layer "F.Cu") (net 8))
 (segment (start 96.8650 26.2000) (end 96.8650 36.9850) (width 0.25) (layer "F.Cu") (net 8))
 (gr_line (start 23.0000 20.0000) (end 113.2000 20.0000) (stroke (width 0.1) (type solid)) (layer "Edge.Cuts"))
 (gr_line (start 116.2000 23.0000) (end 116.2000 109.2000) (stroke (width 0.1) (type solid)) (layer "Edge.Cuts"))
 (gr_line (start 113.2000 112.2000) (end 23.0000 112.2000) (stroke (width 0.1) (type solid)) (layer "Edge.Cuts"))
 (gr_line (start 20.0000 109.2000) (end 20.0000 23.0000) (stroke (width 0.1) (type solid)) (layer "Edge.Cuts"))
 (gr_arc (start 20.0000 23.0000) (mid 20.8787 20.8787) (end 23.0000 20.0000) (stroke (width 0.1) (type solid)) (layer "Edge.Cuts"))
 (gr_arc (start 113.2000 20.0000) (mid 115.3213 20.8787) (end 116.2000 23.0000) (stroke (width 0.1) (type solid)) (layer "Edge.Cuts"))
 (gr_arc (start 116.2000 109.2000) (mid 115.3213 111.3213) (end 113.2000 112.2000) (stroke (width 0.1) (type solid)) (layer "Edge.Cuts"))
 (gr_arc (start 23.0000 112.2000) (mid 20.8787 111.3213) (end 20.0000 109.2000) (stroke (width 0.1) (type solid)) (layer "Edge.Cuts")))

